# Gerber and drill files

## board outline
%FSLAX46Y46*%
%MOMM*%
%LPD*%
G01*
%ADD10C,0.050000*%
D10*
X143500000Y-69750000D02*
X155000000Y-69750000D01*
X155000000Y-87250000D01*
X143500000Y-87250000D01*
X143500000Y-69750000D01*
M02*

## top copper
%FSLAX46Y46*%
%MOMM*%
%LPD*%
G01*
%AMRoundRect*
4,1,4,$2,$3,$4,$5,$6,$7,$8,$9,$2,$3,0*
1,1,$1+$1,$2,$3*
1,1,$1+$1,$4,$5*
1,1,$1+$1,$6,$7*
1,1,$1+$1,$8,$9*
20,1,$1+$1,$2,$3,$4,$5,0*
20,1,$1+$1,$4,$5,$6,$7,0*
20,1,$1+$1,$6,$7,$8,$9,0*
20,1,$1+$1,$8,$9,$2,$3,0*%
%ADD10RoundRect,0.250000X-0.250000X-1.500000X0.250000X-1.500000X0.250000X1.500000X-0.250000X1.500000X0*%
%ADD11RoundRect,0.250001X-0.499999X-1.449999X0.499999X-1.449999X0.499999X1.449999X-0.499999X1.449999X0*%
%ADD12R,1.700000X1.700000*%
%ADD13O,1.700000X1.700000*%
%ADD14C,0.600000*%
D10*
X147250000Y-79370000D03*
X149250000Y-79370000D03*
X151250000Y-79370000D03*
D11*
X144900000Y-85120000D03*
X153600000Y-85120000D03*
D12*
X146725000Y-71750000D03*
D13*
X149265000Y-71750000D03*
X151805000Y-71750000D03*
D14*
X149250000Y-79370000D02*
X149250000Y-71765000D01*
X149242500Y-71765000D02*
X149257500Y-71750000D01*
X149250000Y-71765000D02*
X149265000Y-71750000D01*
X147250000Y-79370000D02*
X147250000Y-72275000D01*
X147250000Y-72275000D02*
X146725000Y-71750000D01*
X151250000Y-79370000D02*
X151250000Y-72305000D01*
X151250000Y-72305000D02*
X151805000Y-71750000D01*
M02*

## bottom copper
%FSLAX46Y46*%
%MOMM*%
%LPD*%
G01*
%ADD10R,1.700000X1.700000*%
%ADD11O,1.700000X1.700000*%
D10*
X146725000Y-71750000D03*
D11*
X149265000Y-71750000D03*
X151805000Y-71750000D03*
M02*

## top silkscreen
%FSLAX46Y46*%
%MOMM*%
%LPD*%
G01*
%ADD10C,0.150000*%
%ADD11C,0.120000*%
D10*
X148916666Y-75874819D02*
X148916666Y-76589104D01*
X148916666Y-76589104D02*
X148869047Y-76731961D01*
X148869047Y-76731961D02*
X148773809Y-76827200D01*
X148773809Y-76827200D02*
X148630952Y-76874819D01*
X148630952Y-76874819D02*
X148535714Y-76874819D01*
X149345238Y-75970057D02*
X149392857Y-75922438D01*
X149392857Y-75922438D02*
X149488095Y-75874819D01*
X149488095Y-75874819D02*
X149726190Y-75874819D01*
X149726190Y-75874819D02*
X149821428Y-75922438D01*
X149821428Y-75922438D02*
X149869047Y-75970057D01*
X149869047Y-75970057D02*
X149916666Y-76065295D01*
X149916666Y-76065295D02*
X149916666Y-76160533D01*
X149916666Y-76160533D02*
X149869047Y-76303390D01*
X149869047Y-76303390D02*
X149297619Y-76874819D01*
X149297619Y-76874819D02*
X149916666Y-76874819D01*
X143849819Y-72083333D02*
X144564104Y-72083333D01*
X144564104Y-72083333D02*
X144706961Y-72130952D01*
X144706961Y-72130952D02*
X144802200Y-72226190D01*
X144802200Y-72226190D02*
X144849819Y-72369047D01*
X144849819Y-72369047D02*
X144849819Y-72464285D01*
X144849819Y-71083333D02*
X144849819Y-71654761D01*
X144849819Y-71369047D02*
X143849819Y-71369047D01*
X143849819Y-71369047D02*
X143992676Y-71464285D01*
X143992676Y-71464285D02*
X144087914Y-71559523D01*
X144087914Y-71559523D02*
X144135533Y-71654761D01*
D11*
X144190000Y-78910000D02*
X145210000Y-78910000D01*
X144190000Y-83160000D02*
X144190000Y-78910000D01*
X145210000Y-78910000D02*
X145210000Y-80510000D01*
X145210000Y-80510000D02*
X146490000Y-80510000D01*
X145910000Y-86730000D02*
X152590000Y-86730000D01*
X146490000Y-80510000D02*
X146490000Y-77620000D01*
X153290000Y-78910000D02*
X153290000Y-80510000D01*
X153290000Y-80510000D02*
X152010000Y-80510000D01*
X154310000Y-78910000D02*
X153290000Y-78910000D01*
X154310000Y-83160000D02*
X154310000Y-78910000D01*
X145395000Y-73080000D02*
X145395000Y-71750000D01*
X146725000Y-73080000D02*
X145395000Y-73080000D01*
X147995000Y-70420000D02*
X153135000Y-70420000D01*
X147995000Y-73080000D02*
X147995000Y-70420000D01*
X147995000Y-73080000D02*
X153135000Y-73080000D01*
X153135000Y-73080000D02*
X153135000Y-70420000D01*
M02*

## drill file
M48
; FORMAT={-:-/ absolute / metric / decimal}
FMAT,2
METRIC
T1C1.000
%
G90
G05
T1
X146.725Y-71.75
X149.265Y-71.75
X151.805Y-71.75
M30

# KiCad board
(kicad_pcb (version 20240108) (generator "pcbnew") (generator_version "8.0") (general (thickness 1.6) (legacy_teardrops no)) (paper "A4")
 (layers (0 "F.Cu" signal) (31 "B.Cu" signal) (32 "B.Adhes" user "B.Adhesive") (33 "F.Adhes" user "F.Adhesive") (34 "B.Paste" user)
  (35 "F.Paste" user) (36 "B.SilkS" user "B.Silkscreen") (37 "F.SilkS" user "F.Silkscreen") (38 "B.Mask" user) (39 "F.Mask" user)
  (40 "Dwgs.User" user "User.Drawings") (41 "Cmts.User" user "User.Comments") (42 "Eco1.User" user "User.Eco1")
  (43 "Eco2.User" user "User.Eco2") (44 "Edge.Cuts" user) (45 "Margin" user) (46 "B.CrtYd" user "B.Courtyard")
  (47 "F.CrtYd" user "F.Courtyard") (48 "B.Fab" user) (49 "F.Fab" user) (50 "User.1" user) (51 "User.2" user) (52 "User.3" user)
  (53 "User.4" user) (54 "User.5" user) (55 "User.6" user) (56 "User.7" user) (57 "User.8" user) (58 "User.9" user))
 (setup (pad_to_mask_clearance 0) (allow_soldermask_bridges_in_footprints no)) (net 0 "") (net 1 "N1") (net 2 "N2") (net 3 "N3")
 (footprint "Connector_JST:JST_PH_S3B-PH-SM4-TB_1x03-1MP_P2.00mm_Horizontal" (layer "F.Cu") (at 149.25 82.22)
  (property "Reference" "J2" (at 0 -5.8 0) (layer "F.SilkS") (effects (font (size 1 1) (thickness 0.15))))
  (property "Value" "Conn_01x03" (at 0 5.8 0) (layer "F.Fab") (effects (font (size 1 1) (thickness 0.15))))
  (fp_line (start -5.06 -3.31) (end -4.04 -3.31) (stroke (width 0.12) (type solid)) (layer "F.SilkS"))
  (fp_line (start -5.06 0.94) (end -5.06 -3.31) (stroke (width 0.12) (type solid)) (layer "F.SilkS"))
  (fp_line (start -4.04 -3.31) (end -4.04 -1.71) (stroke (width 0.12) (type solid)) (layer "F.SilkS"))
  (fp_line (start -4.04 -1.71) (end -2.76 -1.71) (stroke (width 0.12) (type solid)) (layer "F.SilkS"))
  (fp_line (start -3.34 4.51) (end 3.34 4.51) (stroke (width 0.12) (type solid)) (layer "F.SilkS"))
  (fp_line (start -2.76 -1.71) (end -2.76 -4.6) (stroke (width 0.12) (type solid)) (layer "F.SilkS"))
  (fp_line (start 4.04 -3.31) (end 4.04 -1.71) (stroke (width 0.12) (type solid)) (layer "F.SilkS"))
  (fp_line (start 4.04 -1.71) (end 2.76 -1.71) (stroke (width 0.12) (type solid)) (layer "F.SilkS"))
  (fp_line (start 5.06 -3.31) (end 4.04 -3.31) (stroke (width 0.12) (type solid)) (layer "F.SilkS"))
  (fp_line (start 5.06 0.94) (end 5.06 -3.31) (stroke (width 0.12) (type solid)) (layer "F.SilkS"))
  (pad "1" smd roundrect (at -2 -2.85) (size 1 3.5) (layers "F.Cu" "F.Paste" "F.Mask") (roundrect_rratio 0.25) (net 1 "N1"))
  (pad "2" smd roundrect (at 0 -2.85) (size 1 3.5) (layers "F.Cu" "F.Paste" "F.Mask") (roundrect_rratio 0.25) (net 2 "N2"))
  (pad "3" smd roundrect (at 2 -2.85) (size 1 3.5) (layers "F.Cu" "F.Paste" "F.Mask") (roundrect_rratio 0.25) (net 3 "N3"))
  (pad "MP" smd roundrect (at -4.35 2.9) (size 1.5 3.4) (layers "F.Cu" "F.Paste" "F.Mask") (roundrect_rratio 0.166667))
  (pad "MP" smd roundrect (at 4.35 2.9) (size 1.5 3.4) (layers "F.Cu" "F.Paste" "F.Mask") (roundrect_rratio 0.166667)))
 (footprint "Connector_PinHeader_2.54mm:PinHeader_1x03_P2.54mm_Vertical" (layer "F.Cu") (at 146.725 71.75 90)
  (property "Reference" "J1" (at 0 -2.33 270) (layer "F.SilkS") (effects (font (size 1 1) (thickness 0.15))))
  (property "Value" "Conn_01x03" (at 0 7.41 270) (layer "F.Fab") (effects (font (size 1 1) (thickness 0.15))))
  (fp_line (start -1.33 -1.33) (end 0 -1.33) (stroke (width 0.12) (type solid)) (layer "F.SilkS"))
  (fp_line (start -1.33 0) (end -1.33 -1.33) (stroke (width 0.12) (type solid)) (layer "F.SilkS"))
  (fp_line (start 1.33 1.27) (end 1.33 6.41) (stroke (width 0.12) (type solid)) (layer "F.SilkS"))
  (fp_line (start -1.33 1.27) (end 1.33 1.27) (stroke (width 0.12) (type solid)) (layer "F.SilkS"))
  (fp_line (start -1.33 1.27) (end -1.33 6.41) (stroke (width 0.12) (type solid)) (layer "F.SilkS"))
  (fp_line (start -1.33 6.41) (end 1.33 6.41) (stroke (width 0.12) (type solid)) (layer "F.SilkS"))
  (pad "1" thru_hole rect (at 0 0 90) (size 1.7 1.7) (drill 1) (layers "*.Cu" "*.Mask") (remove_unused_layers no) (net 1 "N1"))
  (pad "2" thru_hole oval (at 0 2.54 90) (size 1.7 1.7) (drill 1) (layers "*.Cu" "*.Mask") (remove_unused_layers no) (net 2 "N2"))
  (pad "3" thru_hole oval (at 0 5.08 90) (size 1.7 1.7) (drill 1) (layers "*.Cu" "*.Mask") (remove_unused_layers no) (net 3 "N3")))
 (gr_rect (start 143.5 69.75) (end 155 87.25) (stroke (width 0.05) (type default)) (fill none) (layer "Edge.Cuts"))
 (segment (start 149.25 79.37) (end 149.25 71.765) (width 0.6) (layer "F.Cu") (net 2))
 (segment (start 149.2425 71.765) (end 149.2575 71.75) (width 0.6) (layer "F.Cu") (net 2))
 (segment (start 149.25 71.765) (end 149.265 71.75) (width 0.6) (layer "F.Cu") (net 2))
 (segment (start 147.25 79.37) (end 147.25 72.275) (width 0.6) (layer "F.Cu") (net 1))
 (segment (start 147.25 72.275) (end 146.725 71.75) (width 0.6) (layer "F.Cu") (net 1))
 (segment (start 151.25 79.37) (end 151.25 72.305) (width 0.6) (layer "F.Cu") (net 3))
 (segment (start 151.25 72.305) (end 151.805 71.75) (width 0.6) (layer "F.Cu") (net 3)))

